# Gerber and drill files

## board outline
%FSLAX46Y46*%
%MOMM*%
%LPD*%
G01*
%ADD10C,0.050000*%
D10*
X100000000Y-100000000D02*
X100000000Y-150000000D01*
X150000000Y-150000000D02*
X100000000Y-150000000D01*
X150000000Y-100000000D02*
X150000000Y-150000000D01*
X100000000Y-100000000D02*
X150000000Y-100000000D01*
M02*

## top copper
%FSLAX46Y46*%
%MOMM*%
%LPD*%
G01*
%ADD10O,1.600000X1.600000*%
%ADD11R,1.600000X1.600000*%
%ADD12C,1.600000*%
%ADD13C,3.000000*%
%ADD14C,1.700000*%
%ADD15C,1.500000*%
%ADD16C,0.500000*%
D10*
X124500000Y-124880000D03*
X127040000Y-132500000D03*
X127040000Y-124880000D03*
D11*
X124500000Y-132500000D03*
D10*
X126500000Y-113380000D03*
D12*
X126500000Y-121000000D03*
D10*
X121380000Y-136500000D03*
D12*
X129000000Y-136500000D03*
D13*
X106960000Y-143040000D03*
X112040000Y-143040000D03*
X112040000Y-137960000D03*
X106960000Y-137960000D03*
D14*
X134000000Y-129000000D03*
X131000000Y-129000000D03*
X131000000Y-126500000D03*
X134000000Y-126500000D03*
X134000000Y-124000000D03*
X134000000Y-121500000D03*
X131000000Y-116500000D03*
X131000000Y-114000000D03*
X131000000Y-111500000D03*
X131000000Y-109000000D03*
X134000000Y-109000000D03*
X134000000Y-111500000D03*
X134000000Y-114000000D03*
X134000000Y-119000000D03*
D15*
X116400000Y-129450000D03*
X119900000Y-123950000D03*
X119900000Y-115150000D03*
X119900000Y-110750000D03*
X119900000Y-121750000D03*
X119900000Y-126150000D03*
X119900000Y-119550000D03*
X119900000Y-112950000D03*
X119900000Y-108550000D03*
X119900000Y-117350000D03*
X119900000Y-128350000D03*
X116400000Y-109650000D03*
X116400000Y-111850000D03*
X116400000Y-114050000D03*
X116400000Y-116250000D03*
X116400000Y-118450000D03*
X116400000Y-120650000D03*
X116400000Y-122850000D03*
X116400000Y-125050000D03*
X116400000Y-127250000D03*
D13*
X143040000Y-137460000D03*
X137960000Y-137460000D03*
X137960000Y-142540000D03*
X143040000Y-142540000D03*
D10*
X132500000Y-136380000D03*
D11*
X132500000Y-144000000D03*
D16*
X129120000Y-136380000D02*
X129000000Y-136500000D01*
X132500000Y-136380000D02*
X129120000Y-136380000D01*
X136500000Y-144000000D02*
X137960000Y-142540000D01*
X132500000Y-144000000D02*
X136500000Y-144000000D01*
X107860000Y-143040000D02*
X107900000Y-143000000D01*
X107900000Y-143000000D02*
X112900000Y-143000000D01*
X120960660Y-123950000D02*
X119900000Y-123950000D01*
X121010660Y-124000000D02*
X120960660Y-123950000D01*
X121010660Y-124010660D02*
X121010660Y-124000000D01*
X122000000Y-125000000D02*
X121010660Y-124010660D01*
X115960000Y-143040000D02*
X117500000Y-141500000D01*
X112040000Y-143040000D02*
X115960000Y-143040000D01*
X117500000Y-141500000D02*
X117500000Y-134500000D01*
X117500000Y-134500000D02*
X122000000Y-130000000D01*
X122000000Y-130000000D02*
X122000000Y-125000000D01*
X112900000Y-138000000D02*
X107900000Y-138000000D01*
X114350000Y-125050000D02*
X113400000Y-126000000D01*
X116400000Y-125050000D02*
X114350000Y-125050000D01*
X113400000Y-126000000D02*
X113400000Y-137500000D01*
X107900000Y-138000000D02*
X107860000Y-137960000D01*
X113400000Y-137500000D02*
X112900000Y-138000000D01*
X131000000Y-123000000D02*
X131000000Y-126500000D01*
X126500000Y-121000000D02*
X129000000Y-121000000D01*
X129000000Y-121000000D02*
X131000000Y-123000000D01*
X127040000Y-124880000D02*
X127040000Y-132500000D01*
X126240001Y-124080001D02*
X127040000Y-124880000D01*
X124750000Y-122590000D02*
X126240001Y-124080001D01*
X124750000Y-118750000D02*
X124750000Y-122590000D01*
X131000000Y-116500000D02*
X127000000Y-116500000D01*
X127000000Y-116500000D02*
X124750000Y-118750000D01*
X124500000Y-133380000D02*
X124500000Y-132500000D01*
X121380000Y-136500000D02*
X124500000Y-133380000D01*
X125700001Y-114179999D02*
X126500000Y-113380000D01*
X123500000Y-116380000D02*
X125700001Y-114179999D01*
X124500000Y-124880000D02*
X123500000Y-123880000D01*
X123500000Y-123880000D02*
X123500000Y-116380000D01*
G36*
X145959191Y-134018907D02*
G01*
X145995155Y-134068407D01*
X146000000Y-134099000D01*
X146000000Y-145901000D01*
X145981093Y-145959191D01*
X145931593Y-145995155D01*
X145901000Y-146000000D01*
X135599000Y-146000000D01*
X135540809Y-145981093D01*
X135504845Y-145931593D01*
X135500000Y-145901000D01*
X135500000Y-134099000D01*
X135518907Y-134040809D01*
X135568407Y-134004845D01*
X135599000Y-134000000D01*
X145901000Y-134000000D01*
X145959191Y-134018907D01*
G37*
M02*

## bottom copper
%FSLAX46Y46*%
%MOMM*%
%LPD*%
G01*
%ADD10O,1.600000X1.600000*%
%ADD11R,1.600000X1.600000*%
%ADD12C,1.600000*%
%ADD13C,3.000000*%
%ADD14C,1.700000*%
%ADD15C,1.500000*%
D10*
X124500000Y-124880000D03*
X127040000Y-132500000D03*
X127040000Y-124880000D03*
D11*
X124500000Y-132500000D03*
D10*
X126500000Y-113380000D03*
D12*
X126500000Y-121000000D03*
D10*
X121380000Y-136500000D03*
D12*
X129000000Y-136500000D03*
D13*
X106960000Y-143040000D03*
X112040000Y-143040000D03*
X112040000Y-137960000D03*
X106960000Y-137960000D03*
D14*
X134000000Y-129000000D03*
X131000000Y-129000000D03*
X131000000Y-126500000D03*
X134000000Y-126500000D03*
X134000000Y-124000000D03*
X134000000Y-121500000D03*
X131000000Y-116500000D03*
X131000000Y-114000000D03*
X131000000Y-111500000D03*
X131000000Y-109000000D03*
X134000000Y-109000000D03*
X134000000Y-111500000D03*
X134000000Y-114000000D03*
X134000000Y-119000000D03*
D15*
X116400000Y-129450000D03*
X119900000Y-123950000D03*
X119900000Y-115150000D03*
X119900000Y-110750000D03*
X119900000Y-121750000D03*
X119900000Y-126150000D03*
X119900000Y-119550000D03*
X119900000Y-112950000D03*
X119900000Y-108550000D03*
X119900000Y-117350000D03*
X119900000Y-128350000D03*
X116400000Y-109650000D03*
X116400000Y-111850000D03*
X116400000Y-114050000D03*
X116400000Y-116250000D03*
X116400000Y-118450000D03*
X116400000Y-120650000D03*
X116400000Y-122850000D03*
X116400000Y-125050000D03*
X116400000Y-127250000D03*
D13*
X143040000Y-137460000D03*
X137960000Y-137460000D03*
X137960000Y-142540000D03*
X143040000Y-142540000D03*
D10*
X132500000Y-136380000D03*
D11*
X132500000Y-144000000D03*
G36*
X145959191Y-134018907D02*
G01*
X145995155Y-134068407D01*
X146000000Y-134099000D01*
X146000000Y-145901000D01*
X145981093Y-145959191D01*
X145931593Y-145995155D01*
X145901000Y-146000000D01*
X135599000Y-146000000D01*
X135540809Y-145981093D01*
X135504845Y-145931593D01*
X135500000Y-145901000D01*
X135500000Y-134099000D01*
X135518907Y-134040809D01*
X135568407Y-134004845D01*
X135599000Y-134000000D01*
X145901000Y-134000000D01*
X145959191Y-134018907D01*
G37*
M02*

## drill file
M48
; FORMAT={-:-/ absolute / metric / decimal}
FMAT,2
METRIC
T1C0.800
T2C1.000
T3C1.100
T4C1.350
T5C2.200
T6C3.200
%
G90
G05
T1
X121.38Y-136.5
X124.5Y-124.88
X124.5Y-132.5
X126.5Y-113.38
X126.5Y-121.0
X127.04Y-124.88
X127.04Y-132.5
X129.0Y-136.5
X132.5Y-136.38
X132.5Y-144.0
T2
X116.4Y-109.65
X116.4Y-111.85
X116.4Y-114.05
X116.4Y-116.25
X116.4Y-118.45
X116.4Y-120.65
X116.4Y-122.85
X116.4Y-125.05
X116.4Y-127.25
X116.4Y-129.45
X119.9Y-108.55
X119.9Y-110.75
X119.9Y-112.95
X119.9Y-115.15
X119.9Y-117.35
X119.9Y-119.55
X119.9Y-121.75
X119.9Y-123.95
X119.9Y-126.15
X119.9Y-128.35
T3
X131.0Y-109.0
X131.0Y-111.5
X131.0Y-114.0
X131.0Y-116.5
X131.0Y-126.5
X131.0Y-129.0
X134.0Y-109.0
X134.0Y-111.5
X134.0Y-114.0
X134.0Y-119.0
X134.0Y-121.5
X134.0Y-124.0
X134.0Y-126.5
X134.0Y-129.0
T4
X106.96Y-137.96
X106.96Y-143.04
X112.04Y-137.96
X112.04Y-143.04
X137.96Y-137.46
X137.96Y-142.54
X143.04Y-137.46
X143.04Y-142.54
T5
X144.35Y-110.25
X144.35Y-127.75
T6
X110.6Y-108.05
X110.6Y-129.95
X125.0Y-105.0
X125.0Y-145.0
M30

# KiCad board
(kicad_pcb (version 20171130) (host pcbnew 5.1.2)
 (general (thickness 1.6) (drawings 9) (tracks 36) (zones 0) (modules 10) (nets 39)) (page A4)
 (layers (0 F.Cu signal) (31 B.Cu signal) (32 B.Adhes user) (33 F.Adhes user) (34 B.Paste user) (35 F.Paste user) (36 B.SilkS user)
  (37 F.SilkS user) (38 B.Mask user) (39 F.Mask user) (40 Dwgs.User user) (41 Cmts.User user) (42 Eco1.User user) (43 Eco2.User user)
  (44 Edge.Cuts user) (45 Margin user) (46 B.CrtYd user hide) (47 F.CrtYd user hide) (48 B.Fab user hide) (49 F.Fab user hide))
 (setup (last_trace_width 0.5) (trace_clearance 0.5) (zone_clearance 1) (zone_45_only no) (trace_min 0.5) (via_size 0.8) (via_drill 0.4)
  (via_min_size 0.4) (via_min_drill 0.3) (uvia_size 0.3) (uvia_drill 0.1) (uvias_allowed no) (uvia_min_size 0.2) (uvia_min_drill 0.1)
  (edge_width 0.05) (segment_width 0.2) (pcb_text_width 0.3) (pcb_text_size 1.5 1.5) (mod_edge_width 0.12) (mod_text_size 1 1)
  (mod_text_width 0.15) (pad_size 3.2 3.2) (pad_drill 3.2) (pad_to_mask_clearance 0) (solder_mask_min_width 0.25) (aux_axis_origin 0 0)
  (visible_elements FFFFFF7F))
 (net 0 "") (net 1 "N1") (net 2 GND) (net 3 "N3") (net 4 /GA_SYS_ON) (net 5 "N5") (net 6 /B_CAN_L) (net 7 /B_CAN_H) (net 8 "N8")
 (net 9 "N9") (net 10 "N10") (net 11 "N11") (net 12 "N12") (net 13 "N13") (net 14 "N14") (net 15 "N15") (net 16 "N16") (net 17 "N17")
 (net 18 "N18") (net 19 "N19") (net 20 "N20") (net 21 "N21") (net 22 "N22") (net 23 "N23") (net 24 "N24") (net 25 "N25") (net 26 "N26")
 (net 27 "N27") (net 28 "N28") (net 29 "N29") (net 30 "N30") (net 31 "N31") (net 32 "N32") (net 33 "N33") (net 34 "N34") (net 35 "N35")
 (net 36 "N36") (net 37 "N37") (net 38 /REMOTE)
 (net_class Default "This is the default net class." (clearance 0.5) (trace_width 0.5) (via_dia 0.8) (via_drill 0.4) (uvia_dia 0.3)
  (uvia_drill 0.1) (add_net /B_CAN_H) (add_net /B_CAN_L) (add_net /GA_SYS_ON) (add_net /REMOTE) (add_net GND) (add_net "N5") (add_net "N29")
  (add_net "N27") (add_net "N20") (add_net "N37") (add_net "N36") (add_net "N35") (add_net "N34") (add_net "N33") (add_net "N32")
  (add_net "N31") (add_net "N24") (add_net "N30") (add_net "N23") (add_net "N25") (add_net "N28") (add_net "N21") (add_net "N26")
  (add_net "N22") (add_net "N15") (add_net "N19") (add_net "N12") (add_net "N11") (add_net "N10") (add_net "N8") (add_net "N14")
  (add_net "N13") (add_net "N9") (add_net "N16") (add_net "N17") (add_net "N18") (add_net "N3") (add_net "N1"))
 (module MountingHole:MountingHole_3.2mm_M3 (layer F.Cu) (at 125 145)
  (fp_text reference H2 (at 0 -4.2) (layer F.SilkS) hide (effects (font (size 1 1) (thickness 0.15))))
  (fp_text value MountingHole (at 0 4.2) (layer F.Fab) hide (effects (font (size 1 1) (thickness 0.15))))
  (pad 1 np_thru_hole circle (at 0 0) (size 3.2 3.2) (drill 3.2) (layers *.Cu *.Mask)))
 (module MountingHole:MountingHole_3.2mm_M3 (layer F.Cu) (at 125 105)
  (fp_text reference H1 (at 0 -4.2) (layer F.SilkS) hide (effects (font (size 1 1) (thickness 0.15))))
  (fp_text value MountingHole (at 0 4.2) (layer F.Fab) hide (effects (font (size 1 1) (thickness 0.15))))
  (pad 1 np_thru_hole circle (at 0 0) (size 3.2 3.2) (drill 3.2) (layers *.Cu *.Mask)))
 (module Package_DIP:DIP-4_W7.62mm (layer F.Cu) (at 124.5 132.5 90)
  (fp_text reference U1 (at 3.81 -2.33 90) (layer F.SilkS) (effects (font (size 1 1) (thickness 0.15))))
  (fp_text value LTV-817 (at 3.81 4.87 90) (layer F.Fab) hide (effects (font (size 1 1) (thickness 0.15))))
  (pad 4 thru_hole oval (at 7.62 0 90) (size 1.6 1.6) (drill 0.8) (layers *.Cu *.Mask) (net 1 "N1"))
  (pad 2 thru_hole oval (at 0 2.54 90) (size 1.6 1.6) (drill 0.8) (layers *.Cu *.Mask) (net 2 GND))
  (pad 3 thru_hole oval (at 7.62 2.54 90) (size 1.6 1.6) (drill 0.8) (layers *.Cu *.Mask) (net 2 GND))
  (pad 1 thru_hole rect (at 0 0 90) (size 1.6 1.6) (drill 0.8) (layers *.Cu *.Mask) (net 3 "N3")))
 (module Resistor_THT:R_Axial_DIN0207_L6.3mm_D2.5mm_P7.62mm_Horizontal (layer F.Cu) (at 126.5 121 90)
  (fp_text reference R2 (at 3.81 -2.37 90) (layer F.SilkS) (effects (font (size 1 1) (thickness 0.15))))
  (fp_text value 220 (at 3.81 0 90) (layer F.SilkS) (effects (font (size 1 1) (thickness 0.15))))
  (pad 2 thru_hole oval (at 7.62 0 90) (size 1.6 1.6) (drill 0.8) (layers *.Cu *.Mask) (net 1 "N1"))
  (pad 1 thru_hole circle (at 0 0 90) (size 1.6 1.6) (drill 0.8) (layers *.Cu *.Mask) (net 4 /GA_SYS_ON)))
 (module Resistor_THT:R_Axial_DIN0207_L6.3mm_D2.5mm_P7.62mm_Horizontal (layer F.Cu) (at 129 136.5 180)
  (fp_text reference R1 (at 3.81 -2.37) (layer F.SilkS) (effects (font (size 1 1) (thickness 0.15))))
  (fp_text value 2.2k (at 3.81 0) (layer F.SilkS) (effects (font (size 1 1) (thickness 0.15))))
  (pad 2 thru_hole oval (at 7.62 0 180) (size 1.6 1.6) (drill 0.8) (layers *.Cu *.Mask) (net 3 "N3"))
  (pad 1 thru_hole circle (at 0 0 180) (size 1.6 1.6) (drill 0.8) (layers *.Cu *.Mask) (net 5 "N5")))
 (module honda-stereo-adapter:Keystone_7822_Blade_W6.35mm (layer F.Cu) (at 109.5 140.5 180)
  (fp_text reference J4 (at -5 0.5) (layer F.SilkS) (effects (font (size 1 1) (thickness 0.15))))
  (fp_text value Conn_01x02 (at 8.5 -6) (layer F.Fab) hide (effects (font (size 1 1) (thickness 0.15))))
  (pad 1 thru_hole circle (at 2.54 -2.54 180) (size 3 3) (drill 1.35) (layers *.Cu *.Mask) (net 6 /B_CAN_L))
  (pad 1 thru_hole circle (at -2.54 -2.54 180) (size 3 3) (drill 1.35) (layers *.Cu *.Mask) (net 6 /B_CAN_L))
  (pad 2 thru_hole circle (at -2.54 2.54 180) (size 3 3) (drill 1.35) (layers *.Cu *.Mask) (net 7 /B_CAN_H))
  (pad 2 thru_hole circle (at 2.54 2.54 180) (size 3 3) (drill 1.35) (layers *.Cu *.Mask) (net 7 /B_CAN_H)))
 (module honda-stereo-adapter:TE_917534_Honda (layer F.Cu) (at 134 119)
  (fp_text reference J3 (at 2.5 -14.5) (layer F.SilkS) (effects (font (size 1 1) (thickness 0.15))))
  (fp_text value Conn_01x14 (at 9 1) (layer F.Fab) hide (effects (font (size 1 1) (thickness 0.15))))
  (pad "" np_thru_hole circle (at 10.35 8.75) (size 2.2 2.2) (drill 2.2) (layers *.Cu *.Mask))
  (pad "" np_thru_hole circle (at 10.35 -8.75) (size 2.2 2.2) (drill 2.2) (layers *.Cu *.Mask))
  (pad 14 thru_hole circle (at 0 10) (size 1.7 1.7) (drill 1.1) (layers *.Cu *.Mask) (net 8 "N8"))
  (pad 6 thru_hole circle (at -3 10) (size 1.7 1.7) (drill 1.1) (layers *.Cu *.Mask) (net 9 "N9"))
  (pad 5 thru_hole circle (at -3 7.5) (size 1.7 1.7) (drill 1.1) (layers *.Cu *.Mask) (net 4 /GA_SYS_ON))
  (pad 13 thru_hole circle (at 0 7.5) (size 1.7 1.7) (drill 1.1) (layers *.Cu *.Mask) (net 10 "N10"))
  (pad 12 thru_hole circle (at 0 5) (size 1.7 1.7) (drill 1.1) (layers *.Cu *.Mask) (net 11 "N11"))
  (pad 11 thru_hole circle (at 0 2.5) (size 1.7 1.7) (drill 1.1) (layers *.Cu *.Mask) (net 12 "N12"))
  (pad 4 thru_hole circle (at -3 -2.5) (size 1.7 1.7) (drill 1.1) (layers *.Cu *.Mask) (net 2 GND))
  (pad 3 thru_hole circle (at -3 -5) (size 1.7 1.7) (drill 1.1) (layers *.Cu *.Mask) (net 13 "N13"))
  (pad 2 thru_hole circle (at -3 -7.5) (size 1.7 1.7) (drill 1.1) (layers *.Cu *.Mask) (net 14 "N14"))
  (pad 1 thru_hole circle (at -3 -10) (size 1.7 1.7) (drill 1.1) (layers *.Cu *.Mask) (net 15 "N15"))
  (pad 7 thru_hole circle (at 0 -10) (size 1.7 1.7) (drill 1.1) (layers *.Cu *.Mask) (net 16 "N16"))
  (pad 8 thru_hole circle (at 0 -7.5) (size 1.7 1.7) (drill 1.1) (layers *.Cu *.Mask) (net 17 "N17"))
  (pad 9 thru_hole circle (at 0 -5) (size 1.7 1.7) (drill 1.1) (layers *.Cu *.Mask) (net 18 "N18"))
  (pad 10 thru_hole circle (at 0 0) (size 1.7 1.7) (drill 1.1) (layers *.Cu *.Mask) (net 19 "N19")))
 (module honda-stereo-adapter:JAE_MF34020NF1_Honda (layer F.Cu) (at 116.4 119 180)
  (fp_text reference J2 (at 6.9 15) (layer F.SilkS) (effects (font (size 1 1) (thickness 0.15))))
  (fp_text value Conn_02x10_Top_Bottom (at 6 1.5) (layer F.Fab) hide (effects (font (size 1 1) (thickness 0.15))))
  (pad 11 thru_hole circle (at 0 -10.45 180) (size 1.5 1.5) (drill 1) (layers *.Cu *.Mask) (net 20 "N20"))
  (pad "" np_thru_hole circle (at 5.8 10.95 180) (size 3.2 3.2) (drill 3.2) (layers *.Cu *.Mask))
  (pad 3 thru_hole circle (at -3.5 -4.95 180) (size 1.5 1.5) (drill 1) (layers *.Cu *.Mask) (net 6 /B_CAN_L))
  (pad 7 thru_hole circle (at -3.5 3.85 180) (size 1.5 1.5) (drill 1) (layers *.Cu *.Mask) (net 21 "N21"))
  (pad 9 thru_hole circle (at -3.5 8.25 180) (size 1.5 1.5) (drill 1) (layers *.Cu *.Mask) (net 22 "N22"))
  (pad 4 thru_hole circle (at -3.5 -2.75 180) (size 1.5 1.5) (drill 1) (layers *.Cu *.Mask) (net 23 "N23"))
  (pad 2 thru_hole circle (at -3.5 -7.15 180) (size 1.5 1.5) (drill 1) (layers *.Cu *.Mask) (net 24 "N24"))
  (pad 5 thru_hole circle (at -3.5 -0.55 180) (size 1.5 1.5) (drill 1) (layers *.Cu *.Mask) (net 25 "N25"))
  (pad 8 thru_hole circle (at -3.5 6.05 180) (size 1.5 1.5) (drill 1) (layers *.Cu *.Mask) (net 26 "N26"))
  (pad 10 thru_hole circle (at -3.5 10.45 180) (size 1.5 1.5) (drill 1) (layers *.Cu *.Mask) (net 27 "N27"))
  (pad 6 thru_hole circle (at -3.5 1.65 180) (size 1.5 1.5) (drill 1) (layers *.Cu *.Mask) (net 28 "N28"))
  (pad 1 thru_hole circle (at -3.5 -9.35 180) (size 1.5 1.5) (drill 1) (layers *.Cu *.Mask) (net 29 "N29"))
  (pad 20 thru_hole circle (at 0 9.35 180) (size 1.5 1.5) (drill 1) (layers *.Cu *.Mask) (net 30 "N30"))
  (pad 19 thru_hole circle (at 0 7.15 180) (size 1.5 1.5) (drill 1) (layers *.Cu *.Mask) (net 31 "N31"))
  (pad 18 thru_hole circle (at 0 4.95 180) (size 1.5 1.5) (drill 1) (layers *.Cu *.Mask) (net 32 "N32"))
  (pad 17 thru_hole circle (at 0 2.75 180) (size 1.5 1.5) (drill 1) (layers *.Cu *.Mask) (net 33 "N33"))
  (pad 16 thru_hole circle (at 0 0.55 180) (size 1.5 1.5) (drill 1) (layers *.Cu *.Mask) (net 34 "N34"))
  (pad 15 thru_hole circle (at 0 -1.65 180) (size 1.5 1.5) (drill 1) (layers *.Cu *.Mask) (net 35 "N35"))
  (pad 14 thru_hole circle (at 0 -3.85 180) (size 1.5 1.5) (drill 1) (layers *.Cu *.Mask) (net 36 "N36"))
  (pad 13 thru_hole circle (at 0 -6.05 180) (size 1.5 1.5) (drill 1) (layers *.Cu *.Mask) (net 7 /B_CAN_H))
  (pad 12 thru_hole circle (at 0 -8.25 180) (size 1.5 1.5) (drill 1) (layers *.Cu *.Mask) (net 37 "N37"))
  (pad "" np_thru_hole circle (at 5.8 -10.95 180) (size 3.2 3.2) (drill 3.2) (layers *.Cu *.Mask)))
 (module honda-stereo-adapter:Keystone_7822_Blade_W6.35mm (layer F.Cu) (at 140.5 140)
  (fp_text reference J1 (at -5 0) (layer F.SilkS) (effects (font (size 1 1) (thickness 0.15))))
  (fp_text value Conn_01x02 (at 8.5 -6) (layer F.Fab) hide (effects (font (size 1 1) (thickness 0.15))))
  (pad 1 thru_hole circle (at 2.54 -2.54) (size 3 3) (drill 1.35) (layers *.Cu *.Mask) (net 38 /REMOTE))
  (pad 1 thru_hole circle (at -2.54 -2.54) (size 3 3) (drill 1.35) (layers *.Cu *.Mask) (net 38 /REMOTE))
  (pad 2 thru_hole circle (at -2.54 2.54) (size 3 3) (drill 1.35) (layers *.Cu *.Mask) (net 38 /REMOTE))
  (pad 2 thru_hole circle (at 2.54 2.54) (size 3 3) (drill 1.35) (layers *.Cu *.Mask) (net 38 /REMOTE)))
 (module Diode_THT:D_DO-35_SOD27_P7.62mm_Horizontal (layer F.Cu) (at 132.5 144 90)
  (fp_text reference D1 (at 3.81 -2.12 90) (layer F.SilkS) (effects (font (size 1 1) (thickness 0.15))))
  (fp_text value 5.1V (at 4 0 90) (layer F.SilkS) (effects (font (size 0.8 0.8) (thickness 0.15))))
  (pad 2 thru_hole oval (at 7.62 0 90) (size 1.6 1.6) (drill 0.8) (layers *.Cu *.Mask) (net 5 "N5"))
  (pad 1 thru_hole rect (at 0 0 90) (size 1.6 1.6) (drill 0.8) (layers *.Cu *.Mask) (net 38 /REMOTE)))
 (gr_line (start 100 100) (end 100 150) (layer Edge.Cuts) (width 0.05))
 (gr_line (start 150 150) (end 100 150) (layer Edge.Cuts) (width 0.05))
 (gr_line (start 150 100) (end 150 150) (layer Edge.Cuts) (width 0.05))
 (gr_line (start 100 100) (end 150 100) (layer Edge.Cuts) (width 0.05))
 (segment (start 129.12 136.38) (end 129 136.5) (width 0.5) (layer F.Cu) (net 5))
 (segment (start 132.5 136.38) (end 129.12 136.38) (width 0.5) (layer F.Cu) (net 5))
 (segment (start 136.5 144) (end 137.96 142.54) (width 0.5) (layer F.Cu) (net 38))
 (segment (start 132.5 144) (end 136.5 144) (width 0.5) (layer F.Cu) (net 38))
 (segment (start 107.86 143.04) (end 107.9 143) (width 0.5) (layer F.Cu) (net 6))
 (segment (start 107.9 143) (end 112.9 143) (width 0.5) (layer F.Cu) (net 6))
 (segment (start 120.96066 123.95) (end 119.9 123.95) (width 0.5) (layer F.Cu) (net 6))
 (segment (start 121.01066 124) (end 120.96066 123.95) (width 0.5) (layer F.Cu) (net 6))
 (segment (start 121.01066 124.01066) (end 121.01066 124) (width 0.5) (layer F.Cu) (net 6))
 (segment (start 122 125) (end 121.01066 124.01066) (width 0.5) (layer F.Cu) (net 6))
 (segment (start 115.96 143.04) (end 117.5 141.5) (width 0.5) (layer F.Cu) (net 6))
 (segment (start 112.04 143.04) (end 115.96 143.04) (width 0.5) (layer F.Cu) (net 6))
 (segment (start 117.5 141.5) (end 117.5 134.5) (width 0.5) (layer F.Cu) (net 6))
 (segment (start 117.5 134.5) (end 122 130) (width 0.5) (layer F.Cu) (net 6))
 (segment (start 122 130) (end 122 125) (width 0.5) (layer F.Cu) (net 6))
 (segment (start 112.9 138) (end 107.9 138) (width 0.5) (layer F.Cu) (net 7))
 (segment (start 114.35 125.05) (end 113.4 126) (width 0.5) (layer F.Cu) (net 7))
 (segment (start 116.4 125.05) (end 114.35 125.05) (width 0.5) (layer F.Cu) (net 7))
 (segment (start 113.4 126) (end 113.4 137.5) (width 0.5) (layer F.Cu) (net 7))
 (segment (start 107.9 138) (end 107.86 137.96) (width 0.5) (layer F.Cu) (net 7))
 (segment (start 113.4 137.5) (end 112.9 138) (width 0.5) (layer F.Cu) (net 7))
 (segment (start 131 123) (end 131 126.5) (width 0.5) (layer F.Cu) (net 4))
 (segment (start 126.5 121) (end 129 121) (width 0.5) (layer F.Cu) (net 4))
 (segment (start 129 121) (end 131 123) (width 0.5) (layer F.Cu) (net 4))
 (segment (start 127.04 124.88) (end 127.04 132.5) (width 0.5) (layer F.Cu) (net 2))
 (segment (start 126.240001 124.080001) (end 127.04 124.88) (width 0.5) (layer F.Cu) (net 2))
 (segment (start 124.75 122.59) (end 126.240001 124.080001) (width 0.5) (layer F.Cu) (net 2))
 (segment (start 124.75 118.75) (end 124.75 122.59) (width 0.5) (layer F.Cu) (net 2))
 (segment (start 131 116.5) (end 127 116.5) (width 0.5) (layer F.Cu) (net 2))
 (segment (start 127 116.5) (end 124.75 118.75) (width 0.5) (layer F.Cu) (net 2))
 (segment (start 124.5 133.38) (end 124.5 132.5) (width 0.5) (layer F.Cu) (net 3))
 (segment (start 121.38 136.5) (end 124.5 133.38) (width 0.5) (layer F.Cu) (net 3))
 (segment (start 125.700001 114.179999) (end 126.5 113.38) (width 0.5) (layer F.Cu) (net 1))
 (segment (start 123.5 116.38) (end 125.700001 114.179999) (width 0.5) (layer F.Cu) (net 1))
 (segment (start 124.5 124.88) (end 123.5 123.88) (width 0.5) (layer F.Cu) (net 1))
 (segment (start 123.5 123.88) (end 123.5 116.38) (width 0.5) (layer F.Cu) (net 1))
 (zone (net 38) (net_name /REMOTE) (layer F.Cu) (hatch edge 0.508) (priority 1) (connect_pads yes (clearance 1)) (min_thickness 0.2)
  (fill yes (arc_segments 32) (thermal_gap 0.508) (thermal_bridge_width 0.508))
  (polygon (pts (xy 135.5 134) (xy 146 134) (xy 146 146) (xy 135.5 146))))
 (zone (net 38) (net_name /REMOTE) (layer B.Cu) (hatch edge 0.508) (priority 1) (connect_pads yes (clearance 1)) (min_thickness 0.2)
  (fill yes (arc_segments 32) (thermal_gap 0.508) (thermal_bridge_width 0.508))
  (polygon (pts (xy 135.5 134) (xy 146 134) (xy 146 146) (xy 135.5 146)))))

